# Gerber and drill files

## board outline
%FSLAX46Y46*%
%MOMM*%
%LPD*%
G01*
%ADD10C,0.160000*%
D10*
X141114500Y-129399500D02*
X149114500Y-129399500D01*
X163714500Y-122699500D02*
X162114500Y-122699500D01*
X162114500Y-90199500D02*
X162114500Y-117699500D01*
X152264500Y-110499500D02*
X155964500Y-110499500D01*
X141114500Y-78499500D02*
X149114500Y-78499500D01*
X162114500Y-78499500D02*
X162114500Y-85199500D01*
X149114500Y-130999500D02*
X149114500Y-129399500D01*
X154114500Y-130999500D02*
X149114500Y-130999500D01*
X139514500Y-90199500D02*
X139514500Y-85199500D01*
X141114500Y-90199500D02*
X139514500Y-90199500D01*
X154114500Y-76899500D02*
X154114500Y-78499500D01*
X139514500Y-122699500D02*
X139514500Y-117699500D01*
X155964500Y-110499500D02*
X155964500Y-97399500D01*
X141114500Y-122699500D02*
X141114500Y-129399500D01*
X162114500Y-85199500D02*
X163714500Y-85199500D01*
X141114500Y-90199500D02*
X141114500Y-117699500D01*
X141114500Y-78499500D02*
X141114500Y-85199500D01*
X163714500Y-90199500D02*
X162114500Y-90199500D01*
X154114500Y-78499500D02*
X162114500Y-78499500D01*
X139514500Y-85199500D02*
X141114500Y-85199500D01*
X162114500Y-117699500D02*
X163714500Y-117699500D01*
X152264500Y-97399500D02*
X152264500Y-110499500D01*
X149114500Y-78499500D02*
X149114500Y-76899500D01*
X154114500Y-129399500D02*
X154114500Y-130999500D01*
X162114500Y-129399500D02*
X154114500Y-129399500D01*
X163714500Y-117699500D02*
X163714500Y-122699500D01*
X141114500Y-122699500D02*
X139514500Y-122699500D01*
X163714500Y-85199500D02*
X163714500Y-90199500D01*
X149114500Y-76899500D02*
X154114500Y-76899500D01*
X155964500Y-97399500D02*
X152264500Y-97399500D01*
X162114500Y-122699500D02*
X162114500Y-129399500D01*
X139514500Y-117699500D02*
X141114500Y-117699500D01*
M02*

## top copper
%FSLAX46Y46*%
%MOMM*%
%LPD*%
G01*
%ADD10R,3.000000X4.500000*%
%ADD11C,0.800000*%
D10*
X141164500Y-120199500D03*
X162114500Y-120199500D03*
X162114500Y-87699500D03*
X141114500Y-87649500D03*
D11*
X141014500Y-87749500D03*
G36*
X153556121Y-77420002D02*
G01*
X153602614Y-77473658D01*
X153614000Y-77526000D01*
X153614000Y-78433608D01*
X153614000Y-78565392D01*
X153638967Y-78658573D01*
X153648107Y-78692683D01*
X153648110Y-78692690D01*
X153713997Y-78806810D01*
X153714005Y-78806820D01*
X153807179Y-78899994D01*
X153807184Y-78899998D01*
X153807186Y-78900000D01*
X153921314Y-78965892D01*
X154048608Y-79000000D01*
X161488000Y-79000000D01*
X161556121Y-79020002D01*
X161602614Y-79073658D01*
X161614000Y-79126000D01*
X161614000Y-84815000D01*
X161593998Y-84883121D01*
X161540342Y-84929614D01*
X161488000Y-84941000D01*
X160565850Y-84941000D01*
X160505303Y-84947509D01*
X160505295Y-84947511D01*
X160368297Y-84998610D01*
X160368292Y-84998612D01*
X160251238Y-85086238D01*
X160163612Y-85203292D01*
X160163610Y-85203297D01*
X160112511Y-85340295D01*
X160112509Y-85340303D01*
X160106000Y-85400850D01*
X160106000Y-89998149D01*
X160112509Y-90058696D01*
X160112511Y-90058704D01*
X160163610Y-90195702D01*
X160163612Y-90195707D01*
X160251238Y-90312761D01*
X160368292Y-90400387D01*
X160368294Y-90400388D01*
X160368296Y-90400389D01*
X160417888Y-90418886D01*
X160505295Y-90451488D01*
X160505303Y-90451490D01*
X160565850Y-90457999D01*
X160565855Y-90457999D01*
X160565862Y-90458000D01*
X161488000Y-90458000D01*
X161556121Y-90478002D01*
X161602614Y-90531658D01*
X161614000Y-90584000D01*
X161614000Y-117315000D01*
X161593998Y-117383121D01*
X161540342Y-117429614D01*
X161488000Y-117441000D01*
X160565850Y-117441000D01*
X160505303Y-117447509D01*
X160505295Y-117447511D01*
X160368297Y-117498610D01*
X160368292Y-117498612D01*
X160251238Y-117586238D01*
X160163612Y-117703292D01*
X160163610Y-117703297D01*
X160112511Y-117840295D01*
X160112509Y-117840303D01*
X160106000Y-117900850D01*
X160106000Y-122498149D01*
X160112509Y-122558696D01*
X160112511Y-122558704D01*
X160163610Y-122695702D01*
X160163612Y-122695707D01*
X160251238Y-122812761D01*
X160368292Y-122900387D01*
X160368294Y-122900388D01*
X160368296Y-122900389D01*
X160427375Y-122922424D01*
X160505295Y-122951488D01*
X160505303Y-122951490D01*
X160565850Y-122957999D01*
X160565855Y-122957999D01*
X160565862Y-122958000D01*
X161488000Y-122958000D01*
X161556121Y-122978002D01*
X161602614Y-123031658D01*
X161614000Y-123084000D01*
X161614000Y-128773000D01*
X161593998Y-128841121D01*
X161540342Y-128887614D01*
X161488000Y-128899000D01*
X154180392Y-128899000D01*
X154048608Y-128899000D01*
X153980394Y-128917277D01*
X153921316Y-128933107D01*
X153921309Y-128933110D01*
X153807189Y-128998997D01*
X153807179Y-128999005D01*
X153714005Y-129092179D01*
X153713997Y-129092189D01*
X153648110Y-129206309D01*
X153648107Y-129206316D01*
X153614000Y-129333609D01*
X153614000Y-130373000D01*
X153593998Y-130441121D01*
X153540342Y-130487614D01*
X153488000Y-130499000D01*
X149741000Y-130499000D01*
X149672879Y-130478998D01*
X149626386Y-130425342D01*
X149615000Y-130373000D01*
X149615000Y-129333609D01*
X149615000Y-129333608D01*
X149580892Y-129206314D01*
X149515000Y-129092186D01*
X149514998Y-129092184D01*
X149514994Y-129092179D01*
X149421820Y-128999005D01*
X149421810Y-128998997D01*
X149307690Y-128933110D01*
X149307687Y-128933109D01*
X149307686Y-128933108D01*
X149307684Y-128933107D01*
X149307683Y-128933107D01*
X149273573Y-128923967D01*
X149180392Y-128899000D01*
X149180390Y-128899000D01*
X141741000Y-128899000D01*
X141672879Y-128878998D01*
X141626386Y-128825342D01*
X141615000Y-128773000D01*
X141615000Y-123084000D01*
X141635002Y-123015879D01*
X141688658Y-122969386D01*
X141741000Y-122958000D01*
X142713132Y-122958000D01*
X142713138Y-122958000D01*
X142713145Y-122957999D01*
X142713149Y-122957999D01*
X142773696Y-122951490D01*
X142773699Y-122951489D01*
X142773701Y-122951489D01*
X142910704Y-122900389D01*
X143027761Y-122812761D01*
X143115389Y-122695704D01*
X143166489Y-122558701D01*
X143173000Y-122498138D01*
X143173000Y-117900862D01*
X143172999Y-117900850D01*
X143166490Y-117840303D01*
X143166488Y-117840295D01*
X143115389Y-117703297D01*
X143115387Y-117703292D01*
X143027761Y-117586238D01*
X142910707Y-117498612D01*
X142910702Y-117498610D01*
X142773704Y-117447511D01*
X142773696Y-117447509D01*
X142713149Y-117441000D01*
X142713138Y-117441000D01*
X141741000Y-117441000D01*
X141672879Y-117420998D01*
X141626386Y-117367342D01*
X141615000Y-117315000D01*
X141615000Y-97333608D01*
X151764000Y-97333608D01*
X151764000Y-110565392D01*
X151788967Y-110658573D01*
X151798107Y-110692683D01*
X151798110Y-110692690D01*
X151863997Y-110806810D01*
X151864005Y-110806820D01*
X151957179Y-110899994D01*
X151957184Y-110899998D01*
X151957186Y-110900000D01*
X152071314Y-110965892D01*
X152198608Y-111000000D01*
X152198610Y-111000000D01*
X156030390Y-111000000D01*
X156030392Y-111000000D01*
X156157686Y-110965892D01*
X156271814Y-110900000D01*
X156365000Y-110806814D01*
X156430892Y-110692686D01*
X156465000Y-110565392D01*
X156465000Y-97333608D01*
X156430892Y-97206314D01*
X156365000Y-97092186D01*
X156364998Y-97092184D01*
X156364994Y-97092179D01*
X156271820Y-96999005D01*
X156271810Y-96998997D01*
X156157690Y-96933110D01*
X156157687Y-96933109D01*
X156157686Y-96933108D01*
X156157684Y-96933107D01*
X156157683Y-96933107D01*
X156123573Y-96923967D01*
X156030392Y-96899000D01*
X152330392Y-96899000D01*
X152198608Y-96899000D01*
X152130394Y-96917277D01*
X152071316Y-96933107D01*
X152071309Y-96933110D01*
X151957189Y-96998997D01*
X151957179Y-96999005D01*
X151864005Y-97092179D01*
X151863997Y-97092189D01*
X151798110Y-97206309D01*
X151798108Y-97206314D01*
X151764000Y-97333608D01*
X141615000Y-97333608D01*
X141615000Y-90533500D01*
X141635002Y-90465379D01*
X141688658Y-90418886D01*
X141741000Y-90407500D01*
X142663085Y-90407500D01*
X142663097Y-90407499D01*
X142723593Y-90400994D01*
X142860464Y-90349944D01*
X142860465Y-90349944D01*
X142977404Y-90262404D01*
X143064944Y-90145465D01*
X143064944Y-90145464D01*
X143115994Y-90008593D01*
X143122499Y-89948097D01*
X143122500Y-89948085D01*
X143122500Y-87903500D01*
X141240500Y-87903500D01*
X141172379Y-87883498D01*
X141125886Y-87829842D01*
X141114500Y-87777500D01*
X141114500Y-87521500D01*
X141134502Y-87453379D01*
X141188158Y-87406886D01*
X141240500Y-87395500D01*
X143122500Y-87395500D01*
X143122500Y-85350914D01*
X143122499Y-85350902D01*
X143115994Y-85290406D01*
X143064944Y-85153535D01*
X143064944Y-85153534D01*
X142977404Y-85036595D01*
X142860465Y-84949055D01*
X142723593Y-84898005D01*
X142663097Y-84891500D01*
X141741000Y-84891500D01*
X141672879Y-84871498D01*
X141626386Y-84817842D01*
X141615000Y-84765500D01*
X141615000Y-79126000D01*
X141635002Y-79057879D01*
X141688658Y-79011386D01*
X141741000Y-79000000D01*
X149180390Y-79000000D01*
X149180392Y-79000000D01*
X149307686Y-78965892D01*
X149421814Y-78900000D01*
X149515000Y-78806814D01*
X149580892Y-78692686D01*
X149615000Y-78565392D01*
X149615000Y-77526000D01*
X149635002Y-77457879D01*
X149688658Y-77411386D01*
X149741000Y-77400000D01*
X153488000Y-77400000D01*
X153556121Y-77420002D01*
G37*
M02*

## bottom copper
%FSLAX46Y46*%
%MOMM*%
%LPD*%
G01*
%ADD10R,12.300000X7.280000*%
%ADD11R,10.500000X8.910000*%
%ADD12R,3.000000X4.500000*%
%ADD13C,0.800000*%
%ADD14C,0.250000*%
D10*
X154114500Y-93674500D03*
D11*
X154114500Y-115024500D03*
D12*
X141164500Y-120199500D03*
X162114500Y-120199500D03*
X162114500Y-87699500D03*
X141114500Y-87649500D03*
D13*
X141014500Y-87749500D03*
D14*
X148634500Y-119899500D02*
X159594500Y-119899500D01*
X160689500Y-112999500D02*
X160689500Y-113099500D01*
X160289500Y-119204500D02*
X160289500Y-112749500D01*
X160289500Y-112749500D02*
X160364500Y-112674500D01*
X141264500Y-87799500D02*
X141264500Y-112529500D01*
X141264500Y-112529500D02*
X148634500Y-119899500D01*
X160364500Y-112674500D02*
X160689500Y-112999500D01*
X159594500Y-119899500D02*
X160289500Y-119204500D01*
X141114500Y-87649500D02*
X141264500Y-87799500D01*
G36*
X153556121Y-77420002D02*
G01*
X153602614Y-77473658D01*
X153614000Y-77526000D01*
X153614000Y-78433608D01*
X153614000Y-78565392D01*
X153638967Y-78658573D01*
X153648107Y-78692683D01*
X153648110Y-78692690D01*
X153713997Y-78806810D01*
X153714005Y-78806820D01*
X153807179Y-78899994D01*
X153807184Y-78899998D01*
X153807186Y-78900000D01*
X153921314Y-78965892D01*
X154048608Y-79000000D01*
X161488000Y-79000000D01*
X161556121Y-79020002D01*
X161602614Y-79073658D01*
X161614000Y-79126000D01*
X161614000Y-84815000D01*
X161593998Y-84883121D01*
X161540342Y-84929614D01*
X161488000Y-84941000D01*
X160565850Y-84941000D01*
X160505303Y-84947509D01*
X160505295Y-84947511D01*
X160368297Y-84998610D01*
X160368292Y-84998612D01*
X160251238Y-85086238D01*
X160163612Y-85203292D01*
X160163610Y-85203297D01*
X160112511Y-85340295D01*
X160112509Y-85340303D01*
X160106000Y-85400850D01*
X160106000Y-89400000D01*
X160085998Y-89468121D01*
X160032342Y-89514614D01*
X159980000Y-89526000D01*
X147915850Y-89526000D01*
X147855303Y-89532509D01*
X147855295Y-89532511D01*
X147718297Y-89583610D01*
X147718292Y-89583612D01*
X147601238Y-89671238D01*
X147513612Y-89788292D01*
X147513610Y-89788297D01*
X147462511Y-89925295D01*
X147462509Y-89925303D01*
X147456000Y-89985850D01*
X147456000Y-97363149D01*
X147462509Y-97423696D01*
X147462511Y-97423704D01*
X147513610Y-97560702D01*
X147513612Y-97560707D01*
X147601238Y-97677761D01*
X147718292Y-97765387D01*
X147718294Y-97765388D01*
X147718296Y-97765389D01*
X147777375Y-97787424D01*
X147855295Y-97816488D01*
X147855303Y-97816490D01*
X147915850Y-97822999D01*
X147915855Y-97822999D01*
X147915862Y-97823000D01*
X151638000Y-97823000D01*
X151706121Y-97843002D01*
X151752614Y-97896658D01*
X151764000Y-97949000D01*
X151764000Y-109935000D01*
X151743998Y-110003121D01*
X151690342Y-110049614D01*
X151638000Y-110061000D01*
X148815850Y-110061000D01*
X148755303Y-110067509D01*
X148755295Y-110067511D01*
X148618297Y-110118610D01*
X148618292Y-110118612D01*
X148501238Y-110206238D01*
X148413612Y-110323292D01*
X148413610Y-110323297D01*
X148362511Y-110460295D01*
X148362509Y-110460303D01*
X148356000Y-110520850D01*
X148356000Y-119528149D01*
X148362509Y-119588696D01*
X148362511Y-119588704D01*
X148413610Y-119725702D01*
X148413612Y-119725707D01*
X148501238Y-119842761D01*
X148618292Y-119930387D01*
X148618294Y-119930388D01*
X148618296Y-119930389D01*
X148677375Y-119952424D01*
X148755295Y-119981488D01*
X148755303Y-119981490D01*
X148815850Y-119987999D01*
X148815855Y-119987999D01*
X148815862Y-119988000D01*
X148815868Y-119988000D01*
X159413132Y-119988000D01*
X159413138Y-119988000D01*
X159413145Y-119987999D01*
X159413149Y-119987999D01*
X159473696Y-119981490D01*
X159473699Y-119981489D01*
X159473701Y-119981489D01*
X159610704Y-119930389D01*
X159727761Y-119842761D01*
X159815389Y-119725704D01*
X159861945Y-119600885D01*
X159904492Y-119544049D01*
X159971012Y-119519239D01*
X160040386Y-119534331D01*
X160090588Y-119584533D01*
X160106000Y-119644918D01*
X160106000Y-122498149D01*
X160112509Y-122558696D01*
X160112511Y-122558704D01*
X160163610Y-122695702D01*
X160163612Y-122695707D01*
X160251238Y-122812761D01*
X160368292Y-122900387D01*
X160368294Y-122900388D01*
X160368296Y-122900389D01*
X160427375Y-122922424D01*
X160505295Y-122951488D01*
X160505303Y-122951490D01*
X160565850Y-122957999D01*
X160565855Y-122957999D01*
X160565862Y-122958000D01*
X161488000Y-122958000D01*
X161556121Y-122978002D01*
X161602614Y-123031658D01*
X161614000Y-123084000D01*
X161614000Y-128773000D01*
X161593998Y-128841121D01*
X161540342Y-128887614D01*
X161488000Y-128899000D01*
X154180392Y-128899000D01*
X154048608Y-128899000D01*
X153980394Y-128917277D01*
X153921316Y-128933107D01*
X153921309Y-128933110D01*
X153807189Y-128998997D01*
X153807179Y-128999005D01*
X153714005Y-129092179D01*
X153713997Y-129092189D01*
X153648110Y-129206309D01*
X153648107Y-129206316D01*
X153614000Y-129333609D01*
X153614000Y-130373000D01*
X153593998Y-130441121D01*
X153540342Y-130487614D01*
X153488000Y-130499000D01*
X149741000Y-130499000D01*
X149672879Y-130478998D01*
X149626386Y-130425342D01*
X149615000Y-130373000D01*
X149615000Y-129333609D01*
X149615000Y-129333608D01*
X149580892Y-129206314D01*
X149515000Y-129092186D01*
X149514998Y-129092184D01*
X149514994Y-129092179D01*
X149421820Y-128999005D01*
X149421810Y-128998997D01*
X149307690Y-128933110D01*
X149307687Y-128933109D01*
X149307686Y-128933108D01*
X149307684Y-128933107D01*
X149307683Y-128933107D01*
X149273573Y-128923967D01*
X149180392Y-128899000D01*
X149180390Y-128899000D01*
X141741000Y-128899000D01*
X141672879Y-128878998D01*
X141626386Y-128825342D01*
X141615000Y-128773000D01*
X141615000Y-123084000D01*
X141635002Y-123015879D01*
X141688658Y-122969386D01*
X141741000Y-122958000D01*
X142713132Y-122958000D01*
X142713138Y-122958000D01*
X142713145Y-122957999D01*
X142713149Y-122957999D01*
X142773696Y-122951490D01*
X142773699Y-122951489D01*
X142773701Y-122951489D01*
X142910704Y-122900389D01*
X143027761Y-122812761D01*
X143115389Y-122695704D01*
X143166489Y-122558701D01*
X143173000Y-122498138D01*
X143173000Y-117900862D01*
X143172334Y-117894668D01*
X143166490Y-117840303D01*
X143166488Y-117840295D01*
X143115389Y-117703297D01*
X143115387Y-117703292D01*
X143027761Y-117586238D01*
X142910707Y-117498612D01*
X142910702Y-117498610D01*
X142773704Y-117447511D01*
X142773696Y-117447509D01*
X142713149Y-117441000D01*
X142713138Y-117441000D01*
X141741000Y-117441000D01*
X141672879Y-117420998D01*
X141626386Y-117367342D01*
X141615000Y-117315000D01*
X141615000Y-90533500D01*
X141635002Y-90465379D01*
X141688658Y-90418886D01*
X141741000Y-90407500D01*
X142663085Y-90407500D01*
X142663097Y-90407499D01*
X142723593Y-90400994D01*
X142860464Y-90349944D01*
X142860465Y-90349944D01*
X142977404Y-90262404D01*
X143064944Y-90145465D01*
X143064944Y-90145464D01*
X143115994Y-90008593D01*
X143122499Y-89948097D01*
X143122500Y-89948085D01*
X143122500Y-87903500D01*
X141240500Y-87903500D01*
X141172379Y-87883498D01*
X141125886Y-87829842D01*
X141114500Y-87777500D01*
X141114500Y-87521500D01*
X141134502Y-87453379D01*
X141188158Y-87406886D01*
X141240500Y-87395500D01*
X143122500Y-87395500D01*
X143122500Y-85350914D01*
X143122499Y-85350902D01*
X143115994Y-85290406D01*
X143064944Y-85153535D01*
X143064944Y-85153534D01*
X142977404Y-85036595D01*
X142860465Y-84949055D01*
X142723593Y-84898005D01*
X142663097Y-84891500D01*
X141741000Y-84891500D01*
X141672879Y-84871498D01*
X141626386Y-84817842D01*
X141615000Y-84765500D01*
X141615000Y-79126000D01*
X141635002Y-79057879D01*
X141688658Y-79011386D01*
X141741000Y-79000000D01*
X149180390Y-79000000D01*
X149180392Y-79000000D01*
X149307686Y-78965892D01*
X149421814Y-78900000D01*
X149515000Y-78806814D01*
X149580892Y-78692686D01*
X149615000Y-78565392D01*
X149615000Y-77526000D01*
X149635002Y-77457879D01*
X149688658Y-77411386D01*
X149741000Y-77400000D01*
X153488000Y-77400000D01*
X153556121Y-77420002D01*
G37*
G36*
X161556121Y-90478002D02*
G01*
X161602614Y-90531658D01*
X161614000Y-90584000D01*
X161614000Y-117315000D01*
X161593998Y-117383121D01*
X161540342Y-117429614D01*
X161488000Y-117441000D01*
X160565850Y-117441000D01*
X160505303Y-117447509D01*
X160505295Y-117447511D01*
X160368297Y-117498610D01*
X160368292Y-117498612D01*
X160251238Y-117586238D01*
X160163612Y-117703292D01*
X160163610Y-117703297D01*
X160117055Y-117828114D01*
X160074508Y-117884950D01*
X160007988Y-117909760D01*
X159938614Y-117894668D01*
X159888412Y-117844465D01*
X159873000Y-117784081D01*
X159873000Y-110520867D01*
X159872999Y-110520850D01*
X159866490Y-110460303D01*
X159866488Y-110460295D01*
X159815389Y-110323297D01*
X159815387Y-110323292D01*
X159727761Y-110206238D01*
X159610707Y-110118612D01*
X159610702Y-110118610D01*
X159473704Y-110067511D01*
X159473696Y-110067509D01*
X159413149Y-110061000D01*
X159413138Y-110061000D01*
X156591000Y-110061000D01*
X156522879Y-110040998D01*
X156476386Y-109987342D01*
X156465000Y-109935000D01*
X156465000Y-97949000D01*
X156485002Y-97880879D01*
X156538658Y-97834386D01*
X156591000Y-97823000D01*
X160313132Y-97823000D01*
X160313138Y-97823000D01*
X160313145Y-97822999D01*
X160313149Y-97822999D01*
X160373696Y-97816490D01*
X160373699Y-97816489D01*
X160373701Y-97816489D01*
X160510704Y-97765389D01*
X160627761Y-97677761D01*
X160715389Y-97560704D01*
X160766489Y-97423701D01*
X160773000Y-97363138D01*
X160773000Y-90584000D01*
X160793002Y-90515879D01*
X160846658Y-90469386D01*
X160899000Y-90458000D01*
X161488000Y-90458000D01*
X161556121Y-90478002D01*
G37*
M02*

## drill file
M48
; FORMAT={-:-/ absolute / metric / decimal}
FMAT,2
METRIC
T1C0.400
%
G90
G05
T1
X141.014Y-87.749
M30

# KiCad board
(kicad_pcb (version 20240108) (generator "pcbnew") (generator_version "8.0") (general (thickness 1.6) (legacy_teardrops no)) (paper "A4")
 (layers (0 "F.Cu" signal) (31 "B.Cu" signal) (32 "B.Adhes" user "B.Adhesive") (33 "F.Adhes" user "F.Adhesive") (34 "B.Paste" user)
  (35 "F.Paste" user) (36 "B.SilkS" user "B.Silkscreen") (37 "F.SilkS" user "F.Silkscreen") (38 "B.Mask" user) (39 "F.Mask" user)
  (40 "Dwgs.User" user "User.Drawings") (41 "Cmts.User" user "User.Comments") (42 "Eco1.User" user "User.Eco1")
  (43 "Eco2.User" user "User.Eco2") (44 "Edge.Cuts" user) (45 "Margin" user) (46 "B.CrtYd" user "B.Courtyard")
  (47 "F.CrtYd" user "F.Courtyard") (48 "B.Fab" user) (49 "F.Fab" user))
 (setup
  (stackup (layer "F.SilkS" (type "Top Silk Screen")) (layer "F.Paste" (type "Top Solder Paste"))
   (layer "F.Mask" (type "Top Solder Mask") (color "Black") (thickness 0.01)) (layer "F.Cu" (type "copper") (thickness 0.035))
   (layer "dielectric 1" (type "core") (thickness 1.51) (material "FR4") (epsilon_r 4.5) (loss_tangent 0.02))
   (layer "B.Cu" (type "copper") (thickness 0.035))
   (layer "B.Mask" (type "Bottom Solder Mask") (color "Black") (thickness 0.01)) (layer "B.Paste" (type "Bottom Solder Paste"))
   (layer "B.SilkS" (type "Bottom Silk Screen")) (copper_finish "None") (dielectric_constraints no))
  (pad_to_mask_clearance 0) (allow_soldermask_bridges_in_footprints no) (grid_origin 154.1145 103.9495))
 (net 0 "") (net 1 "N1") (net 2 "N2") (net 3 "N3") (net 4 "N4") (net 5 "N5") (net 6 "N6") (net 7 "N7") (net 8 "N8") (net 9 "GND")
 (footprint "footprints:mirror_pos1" (layer "F.Cu") (at 154.1145 93.6745 90)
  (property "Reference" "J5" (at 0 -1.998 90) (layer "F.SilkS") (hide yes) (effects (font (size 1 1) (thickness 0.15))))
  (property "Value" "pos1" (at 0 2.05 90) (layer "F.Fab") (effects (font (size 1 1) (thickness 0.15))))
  (pad "1" smd rect (at 0 0 90) (size 7.28 12.3) (layers "B.Cu" "B.Mask") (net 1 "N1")))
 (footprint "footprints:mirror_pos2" (layer "F.Cu") (at 154.1145 115.0245 90)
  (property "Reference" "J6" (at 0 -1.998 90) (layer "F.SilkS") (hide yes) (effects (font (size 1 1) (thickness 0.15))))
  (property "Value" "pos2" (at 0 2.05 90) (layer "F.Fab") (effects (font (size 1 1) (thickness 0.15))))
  (pad "1" smd rect (at 0 0 90) (size 8.91 10.5) (layers "B.Cu" "B.Mask") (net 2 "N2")))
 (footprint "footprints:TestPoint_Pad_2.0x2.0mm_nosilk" (layer "F.Cu") (at 141.1645 120.1995 90)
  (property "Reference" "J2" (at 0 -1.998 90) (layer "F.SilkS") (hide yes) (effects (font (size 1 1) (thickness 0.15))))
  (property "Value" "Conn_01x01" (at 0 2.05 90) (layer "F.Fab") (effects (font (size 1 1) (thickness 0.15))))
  (pad "1" smd rect (at 0 0 90) (size 4.5 3) (layers "F.Cu" "F.Mask") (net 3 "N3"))
  (pad "1" smd rect (at 0 0 90) (size 4.5 3) (layers "B.Cu" "B.Mask") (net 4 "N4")))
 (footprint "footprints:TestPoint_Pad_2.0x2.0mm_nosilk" (layer "F.Cu") (at 162.1145 120.1995 90)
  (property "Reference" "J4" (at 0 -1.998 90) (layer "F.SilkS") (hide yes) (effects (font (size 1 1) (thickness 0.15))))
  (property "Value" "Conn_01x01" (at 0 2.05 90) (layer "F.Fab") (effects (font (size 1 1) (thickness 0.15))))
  (pad "1" smd rect (at 0 0 90) (size 4.5 3) (layers "F.Cu" "F.Mask") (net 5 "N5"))
  (pad "1" smd rect (at 0 0 90) (size 4.5 3) (layers "B.Cu" "B.Mask") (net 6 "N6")))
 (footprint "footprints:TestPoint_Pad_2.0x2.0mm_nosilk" (layer "F.Cu") (at 162.1145 87.6995 90)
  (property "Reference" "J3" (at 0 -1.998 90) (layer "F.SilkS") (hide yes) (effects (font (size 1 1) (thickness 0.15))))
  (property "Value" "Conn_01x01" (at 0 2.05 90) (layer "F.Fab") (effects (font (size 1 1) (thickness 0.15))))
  (pad "1" smd rect (at 0 0 90) (size 4.5 3) (layers "F.Cu" "F.Mask") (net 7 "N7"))
  (pad "1" smd rect (at 0 0 90) (size 4.5 3) (layers "B.Cu" "B.Mask") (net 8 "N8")))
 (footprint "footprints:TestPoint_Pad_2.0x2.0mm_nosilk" (layer "F.Cu") (at 141.1145 87.6495 90)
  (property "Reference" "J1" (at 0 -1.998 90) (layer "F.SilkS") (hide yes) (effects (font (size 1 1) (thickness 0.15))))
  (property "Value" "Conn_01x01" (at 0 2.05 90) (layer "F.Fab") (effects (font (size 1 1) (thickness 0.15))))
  (pad "1" smd rect (at 0 0 90) (size 4.5 3) (layers "F.Cu" "F.Mask") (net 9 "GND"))
  (pad "1" smd rect (at 0 0 90) (size 4.5 3) (layers "B.Cu" "B.Mask") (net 9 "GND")))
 (gr_line (start 141.1145 129.3995) (end 149.1145 129.3995) (stroke (width 0.16) (type solid)) (layer "Edge.Cuts"))
 (gr_line (start 163.7145 122.6995) (end 162.1145 122.6995) (stroke (width 0.16) (type solid)) (layer "Edge.Cuts"))
 (gr_line (start 162.1145 90.1995) (end 162.1145 117.6995) (stroke (width 0.16) (type solid)) (layer "Edge.Cuts"))
 (gr_line (start 152.2645 110.4995) (end 155.9645 110.4995) (stroke (width 0.16) (type solid)) (layer "Edge.Cuts"))
 (gr_line (start 141.1145 78.4995) (end 149.1145 78.4995) (stroke (width 0.16) (type solid)) (layer "Edge.Cuts"))
 (gr_line (start 162.1145 78.4995) (end 162.1145 85.1995) (stroke (width 0.16) (type solid)) (layer "Edge.Cuts"))
 (gr_line (start 149.1145 130.9995) (end 149.1145 129.3995) (stroke (width 0.16) (type solid)) (layer "Edge.Cuts"))
 (gr_line (start 154.1145 130.9995) (end 149.1145 130.9995) (stroke (width 0.16) (type solid)) (layer "Edge.Cuts"))
 (gr_line (start 139.5145 90.1995) (end 139.5145 85.1995) (stroke (width 0.16) (type solid)) (layer "Edge.Cuts"))
 (gr_line (start 141.1145 90.1995) (end 139.5145 90.1995) (stroke (width 0.16) (type solid)) (layer "Edge.Cuts"))
 (gr_line (start 154.1145 76.8995) (end 154.1145 78.4995) (stroke (width 0.16) (type solid)) (layer "Edge.Cuts"))
 (gr_line (start 139.5145 122.6995) (end 139.5145 117.6995) (stroke (width 0.16) (type solid)) (layer "Edge.Cuts"))
 (gr_line (start 155.9645 110.4995) (end 155.9645 97.3995) (stroke (width 0.16) (type solid)) (layer "Edge.Cuts"))
 (gr_line (start 141.1145 122.6995) (end 141.1145 129.3995) (stroke (width 0.16) (type solid)) (layer "Edge.Cuts"))
 (gr_line (start 162.1145 85.1995) (end 163.7145 85.1995) (stroke (width 0.16) (type solid)) (layer "Edge.Cuts"))
 (gr_line (start 141.1145 90.1995) (end 141.1145 117.6995) (stroke (width 0.16) (type solid)) (layer "Edge.Cuts"))
 (gr_line (start 141.1145 78.4995) (end 141.1145 85.1995) (stroke (width 0.16) (type solid)) (layer "Edge.Cuts"))
 (gr_line (start 163.7145 90.1995) (end 162.1145 90.1995) (stroke (width 0.16) (type solid)) (layer "Edge.Cuts"))
 (gr_line (start 154.1145 78.4995) (end 162.1145 78.4995) (stroke (width 0.16) (type solid)) (layer "Edge.Cuts"))
 (gr_line (start 139.5145 85.1995) (end 141.1145 85.1995) (stroke (width 0.16) (type solid)) (layer "Edge.Cuts"))
 (gr_line (start 162.1145 117.6995) (end 163.7145 117.6995) (stroke (width 0.16) (type solid)) (layer "Edge.Cuts"))
 (gr_line (start 152.2645 97.3995) (end 152.2645 110.4995) (stroke (width 0.16) (type solid)) (layer "Edge.Cuts"))
 (gr_line (start 149.1145 78.4995) (end 149.1145 76.8995) (stroke (width 0.16) (type solid)) (layer "Edge.Cuts"))
 (gr_line (start 154.1145 129.3995) (end 154.1145 130.9995) (stroke (width 0.16) (type solid)) (layer "Edge.Cuts"))
 (gr_line (start 162.1145 129.3995) (end 154.1145 129.3995) (stroke (width 0.16) (type solid)) (layer "Edge.Cuts"))
 (gr_line (start 163.7145 117.6995) (end 163.7145 122.6995) (stroke (width 0.16) (type solid)) (layer "Edge.Cuts"))
 (gr_line (start 141.1145 122.6995) (end 139.5145 122.6995) (stroke (width 0.16) (type solid)) (layer "Edge.Cuts"))
 (gr_line (start 163.7145 85.1995) (end 163.7145 90.1995) (stroke (width 0.16) (type solid)) (layer "Edge.Cuts"))
 (gr_line (start 149.1145 76.8995) (end 154.1145 76.8995) (stroke (width 0.16) (type solid)) (layer "Edge.Cuts"))
 (gr_line (start 155.9645 97.3995) (end 152.2645 97.3995) (stroke (width 0.16) (type solid)) (layer "Edge.Cuts"))
 (gr_line (start 162.1145 122.6995) (end 162.1145 129.3995) (stroke (width 0.16) (type solid)) (layer "Edge.Cuts"))
 (gr_line (start 139.5145 117.6995) (end 141.1145 117.6995) (stroke (width 0.16) (type solid)) (layer "Edge.Cuts"))
 (via (at 141.0145 87.7495) (size 0.8) (drill 0.4) (layers "F.Cu" "B.Cu") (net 9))
 (segment (start 148.6345 119.8995) (end 159.5945 119.8995) (width 0.25) (layer "B.Cu") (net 9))
 (segment (start 160.6895 112.9995) (end 160.6895 113.0995) (width 0.25) (layer "B.Cu") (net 9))
 (segment (start 160.2895 119.2045) (end 160.2895 112.7495) (width 0.25) (layer "B.Cu") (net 9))
 (segment (start 160.2895 112.7495) (end 160.3645 112.6745) (width 0.25) (layer "B.Cu") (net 9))
 (segment (start 141.2645 87.7995) (end 141.2645 112.5295) (width 0.25) (layer "B.Cu") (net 9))
 (segment (start 141.2645 112.5295) (end 148.6345 119.8995) (width 0.25) (layer "B.Cu") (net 9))
 (segment (start 160.3645 112.6745) (end 160.6895 112.9995) (width 0.25) (layer "B.Cu") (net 9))
 (segment (start 159.5945 119.8995) (end 160.2895 119.2045) (width 0.25) (layer "B.Cu") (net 9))
 (segment (start 141.1145 87.6495) (end 141.2645 87.7995) (width 0.25) (layer "B.Cu") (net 9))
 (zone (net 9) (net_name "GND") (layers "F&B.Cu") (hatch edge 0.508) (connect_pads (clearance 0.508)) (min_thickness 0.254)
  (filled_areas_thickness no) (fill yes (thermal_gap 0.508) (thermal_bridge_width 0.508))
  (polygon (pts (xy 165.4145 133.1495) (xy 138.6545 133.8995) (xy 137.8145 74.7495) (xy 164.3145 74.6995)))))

